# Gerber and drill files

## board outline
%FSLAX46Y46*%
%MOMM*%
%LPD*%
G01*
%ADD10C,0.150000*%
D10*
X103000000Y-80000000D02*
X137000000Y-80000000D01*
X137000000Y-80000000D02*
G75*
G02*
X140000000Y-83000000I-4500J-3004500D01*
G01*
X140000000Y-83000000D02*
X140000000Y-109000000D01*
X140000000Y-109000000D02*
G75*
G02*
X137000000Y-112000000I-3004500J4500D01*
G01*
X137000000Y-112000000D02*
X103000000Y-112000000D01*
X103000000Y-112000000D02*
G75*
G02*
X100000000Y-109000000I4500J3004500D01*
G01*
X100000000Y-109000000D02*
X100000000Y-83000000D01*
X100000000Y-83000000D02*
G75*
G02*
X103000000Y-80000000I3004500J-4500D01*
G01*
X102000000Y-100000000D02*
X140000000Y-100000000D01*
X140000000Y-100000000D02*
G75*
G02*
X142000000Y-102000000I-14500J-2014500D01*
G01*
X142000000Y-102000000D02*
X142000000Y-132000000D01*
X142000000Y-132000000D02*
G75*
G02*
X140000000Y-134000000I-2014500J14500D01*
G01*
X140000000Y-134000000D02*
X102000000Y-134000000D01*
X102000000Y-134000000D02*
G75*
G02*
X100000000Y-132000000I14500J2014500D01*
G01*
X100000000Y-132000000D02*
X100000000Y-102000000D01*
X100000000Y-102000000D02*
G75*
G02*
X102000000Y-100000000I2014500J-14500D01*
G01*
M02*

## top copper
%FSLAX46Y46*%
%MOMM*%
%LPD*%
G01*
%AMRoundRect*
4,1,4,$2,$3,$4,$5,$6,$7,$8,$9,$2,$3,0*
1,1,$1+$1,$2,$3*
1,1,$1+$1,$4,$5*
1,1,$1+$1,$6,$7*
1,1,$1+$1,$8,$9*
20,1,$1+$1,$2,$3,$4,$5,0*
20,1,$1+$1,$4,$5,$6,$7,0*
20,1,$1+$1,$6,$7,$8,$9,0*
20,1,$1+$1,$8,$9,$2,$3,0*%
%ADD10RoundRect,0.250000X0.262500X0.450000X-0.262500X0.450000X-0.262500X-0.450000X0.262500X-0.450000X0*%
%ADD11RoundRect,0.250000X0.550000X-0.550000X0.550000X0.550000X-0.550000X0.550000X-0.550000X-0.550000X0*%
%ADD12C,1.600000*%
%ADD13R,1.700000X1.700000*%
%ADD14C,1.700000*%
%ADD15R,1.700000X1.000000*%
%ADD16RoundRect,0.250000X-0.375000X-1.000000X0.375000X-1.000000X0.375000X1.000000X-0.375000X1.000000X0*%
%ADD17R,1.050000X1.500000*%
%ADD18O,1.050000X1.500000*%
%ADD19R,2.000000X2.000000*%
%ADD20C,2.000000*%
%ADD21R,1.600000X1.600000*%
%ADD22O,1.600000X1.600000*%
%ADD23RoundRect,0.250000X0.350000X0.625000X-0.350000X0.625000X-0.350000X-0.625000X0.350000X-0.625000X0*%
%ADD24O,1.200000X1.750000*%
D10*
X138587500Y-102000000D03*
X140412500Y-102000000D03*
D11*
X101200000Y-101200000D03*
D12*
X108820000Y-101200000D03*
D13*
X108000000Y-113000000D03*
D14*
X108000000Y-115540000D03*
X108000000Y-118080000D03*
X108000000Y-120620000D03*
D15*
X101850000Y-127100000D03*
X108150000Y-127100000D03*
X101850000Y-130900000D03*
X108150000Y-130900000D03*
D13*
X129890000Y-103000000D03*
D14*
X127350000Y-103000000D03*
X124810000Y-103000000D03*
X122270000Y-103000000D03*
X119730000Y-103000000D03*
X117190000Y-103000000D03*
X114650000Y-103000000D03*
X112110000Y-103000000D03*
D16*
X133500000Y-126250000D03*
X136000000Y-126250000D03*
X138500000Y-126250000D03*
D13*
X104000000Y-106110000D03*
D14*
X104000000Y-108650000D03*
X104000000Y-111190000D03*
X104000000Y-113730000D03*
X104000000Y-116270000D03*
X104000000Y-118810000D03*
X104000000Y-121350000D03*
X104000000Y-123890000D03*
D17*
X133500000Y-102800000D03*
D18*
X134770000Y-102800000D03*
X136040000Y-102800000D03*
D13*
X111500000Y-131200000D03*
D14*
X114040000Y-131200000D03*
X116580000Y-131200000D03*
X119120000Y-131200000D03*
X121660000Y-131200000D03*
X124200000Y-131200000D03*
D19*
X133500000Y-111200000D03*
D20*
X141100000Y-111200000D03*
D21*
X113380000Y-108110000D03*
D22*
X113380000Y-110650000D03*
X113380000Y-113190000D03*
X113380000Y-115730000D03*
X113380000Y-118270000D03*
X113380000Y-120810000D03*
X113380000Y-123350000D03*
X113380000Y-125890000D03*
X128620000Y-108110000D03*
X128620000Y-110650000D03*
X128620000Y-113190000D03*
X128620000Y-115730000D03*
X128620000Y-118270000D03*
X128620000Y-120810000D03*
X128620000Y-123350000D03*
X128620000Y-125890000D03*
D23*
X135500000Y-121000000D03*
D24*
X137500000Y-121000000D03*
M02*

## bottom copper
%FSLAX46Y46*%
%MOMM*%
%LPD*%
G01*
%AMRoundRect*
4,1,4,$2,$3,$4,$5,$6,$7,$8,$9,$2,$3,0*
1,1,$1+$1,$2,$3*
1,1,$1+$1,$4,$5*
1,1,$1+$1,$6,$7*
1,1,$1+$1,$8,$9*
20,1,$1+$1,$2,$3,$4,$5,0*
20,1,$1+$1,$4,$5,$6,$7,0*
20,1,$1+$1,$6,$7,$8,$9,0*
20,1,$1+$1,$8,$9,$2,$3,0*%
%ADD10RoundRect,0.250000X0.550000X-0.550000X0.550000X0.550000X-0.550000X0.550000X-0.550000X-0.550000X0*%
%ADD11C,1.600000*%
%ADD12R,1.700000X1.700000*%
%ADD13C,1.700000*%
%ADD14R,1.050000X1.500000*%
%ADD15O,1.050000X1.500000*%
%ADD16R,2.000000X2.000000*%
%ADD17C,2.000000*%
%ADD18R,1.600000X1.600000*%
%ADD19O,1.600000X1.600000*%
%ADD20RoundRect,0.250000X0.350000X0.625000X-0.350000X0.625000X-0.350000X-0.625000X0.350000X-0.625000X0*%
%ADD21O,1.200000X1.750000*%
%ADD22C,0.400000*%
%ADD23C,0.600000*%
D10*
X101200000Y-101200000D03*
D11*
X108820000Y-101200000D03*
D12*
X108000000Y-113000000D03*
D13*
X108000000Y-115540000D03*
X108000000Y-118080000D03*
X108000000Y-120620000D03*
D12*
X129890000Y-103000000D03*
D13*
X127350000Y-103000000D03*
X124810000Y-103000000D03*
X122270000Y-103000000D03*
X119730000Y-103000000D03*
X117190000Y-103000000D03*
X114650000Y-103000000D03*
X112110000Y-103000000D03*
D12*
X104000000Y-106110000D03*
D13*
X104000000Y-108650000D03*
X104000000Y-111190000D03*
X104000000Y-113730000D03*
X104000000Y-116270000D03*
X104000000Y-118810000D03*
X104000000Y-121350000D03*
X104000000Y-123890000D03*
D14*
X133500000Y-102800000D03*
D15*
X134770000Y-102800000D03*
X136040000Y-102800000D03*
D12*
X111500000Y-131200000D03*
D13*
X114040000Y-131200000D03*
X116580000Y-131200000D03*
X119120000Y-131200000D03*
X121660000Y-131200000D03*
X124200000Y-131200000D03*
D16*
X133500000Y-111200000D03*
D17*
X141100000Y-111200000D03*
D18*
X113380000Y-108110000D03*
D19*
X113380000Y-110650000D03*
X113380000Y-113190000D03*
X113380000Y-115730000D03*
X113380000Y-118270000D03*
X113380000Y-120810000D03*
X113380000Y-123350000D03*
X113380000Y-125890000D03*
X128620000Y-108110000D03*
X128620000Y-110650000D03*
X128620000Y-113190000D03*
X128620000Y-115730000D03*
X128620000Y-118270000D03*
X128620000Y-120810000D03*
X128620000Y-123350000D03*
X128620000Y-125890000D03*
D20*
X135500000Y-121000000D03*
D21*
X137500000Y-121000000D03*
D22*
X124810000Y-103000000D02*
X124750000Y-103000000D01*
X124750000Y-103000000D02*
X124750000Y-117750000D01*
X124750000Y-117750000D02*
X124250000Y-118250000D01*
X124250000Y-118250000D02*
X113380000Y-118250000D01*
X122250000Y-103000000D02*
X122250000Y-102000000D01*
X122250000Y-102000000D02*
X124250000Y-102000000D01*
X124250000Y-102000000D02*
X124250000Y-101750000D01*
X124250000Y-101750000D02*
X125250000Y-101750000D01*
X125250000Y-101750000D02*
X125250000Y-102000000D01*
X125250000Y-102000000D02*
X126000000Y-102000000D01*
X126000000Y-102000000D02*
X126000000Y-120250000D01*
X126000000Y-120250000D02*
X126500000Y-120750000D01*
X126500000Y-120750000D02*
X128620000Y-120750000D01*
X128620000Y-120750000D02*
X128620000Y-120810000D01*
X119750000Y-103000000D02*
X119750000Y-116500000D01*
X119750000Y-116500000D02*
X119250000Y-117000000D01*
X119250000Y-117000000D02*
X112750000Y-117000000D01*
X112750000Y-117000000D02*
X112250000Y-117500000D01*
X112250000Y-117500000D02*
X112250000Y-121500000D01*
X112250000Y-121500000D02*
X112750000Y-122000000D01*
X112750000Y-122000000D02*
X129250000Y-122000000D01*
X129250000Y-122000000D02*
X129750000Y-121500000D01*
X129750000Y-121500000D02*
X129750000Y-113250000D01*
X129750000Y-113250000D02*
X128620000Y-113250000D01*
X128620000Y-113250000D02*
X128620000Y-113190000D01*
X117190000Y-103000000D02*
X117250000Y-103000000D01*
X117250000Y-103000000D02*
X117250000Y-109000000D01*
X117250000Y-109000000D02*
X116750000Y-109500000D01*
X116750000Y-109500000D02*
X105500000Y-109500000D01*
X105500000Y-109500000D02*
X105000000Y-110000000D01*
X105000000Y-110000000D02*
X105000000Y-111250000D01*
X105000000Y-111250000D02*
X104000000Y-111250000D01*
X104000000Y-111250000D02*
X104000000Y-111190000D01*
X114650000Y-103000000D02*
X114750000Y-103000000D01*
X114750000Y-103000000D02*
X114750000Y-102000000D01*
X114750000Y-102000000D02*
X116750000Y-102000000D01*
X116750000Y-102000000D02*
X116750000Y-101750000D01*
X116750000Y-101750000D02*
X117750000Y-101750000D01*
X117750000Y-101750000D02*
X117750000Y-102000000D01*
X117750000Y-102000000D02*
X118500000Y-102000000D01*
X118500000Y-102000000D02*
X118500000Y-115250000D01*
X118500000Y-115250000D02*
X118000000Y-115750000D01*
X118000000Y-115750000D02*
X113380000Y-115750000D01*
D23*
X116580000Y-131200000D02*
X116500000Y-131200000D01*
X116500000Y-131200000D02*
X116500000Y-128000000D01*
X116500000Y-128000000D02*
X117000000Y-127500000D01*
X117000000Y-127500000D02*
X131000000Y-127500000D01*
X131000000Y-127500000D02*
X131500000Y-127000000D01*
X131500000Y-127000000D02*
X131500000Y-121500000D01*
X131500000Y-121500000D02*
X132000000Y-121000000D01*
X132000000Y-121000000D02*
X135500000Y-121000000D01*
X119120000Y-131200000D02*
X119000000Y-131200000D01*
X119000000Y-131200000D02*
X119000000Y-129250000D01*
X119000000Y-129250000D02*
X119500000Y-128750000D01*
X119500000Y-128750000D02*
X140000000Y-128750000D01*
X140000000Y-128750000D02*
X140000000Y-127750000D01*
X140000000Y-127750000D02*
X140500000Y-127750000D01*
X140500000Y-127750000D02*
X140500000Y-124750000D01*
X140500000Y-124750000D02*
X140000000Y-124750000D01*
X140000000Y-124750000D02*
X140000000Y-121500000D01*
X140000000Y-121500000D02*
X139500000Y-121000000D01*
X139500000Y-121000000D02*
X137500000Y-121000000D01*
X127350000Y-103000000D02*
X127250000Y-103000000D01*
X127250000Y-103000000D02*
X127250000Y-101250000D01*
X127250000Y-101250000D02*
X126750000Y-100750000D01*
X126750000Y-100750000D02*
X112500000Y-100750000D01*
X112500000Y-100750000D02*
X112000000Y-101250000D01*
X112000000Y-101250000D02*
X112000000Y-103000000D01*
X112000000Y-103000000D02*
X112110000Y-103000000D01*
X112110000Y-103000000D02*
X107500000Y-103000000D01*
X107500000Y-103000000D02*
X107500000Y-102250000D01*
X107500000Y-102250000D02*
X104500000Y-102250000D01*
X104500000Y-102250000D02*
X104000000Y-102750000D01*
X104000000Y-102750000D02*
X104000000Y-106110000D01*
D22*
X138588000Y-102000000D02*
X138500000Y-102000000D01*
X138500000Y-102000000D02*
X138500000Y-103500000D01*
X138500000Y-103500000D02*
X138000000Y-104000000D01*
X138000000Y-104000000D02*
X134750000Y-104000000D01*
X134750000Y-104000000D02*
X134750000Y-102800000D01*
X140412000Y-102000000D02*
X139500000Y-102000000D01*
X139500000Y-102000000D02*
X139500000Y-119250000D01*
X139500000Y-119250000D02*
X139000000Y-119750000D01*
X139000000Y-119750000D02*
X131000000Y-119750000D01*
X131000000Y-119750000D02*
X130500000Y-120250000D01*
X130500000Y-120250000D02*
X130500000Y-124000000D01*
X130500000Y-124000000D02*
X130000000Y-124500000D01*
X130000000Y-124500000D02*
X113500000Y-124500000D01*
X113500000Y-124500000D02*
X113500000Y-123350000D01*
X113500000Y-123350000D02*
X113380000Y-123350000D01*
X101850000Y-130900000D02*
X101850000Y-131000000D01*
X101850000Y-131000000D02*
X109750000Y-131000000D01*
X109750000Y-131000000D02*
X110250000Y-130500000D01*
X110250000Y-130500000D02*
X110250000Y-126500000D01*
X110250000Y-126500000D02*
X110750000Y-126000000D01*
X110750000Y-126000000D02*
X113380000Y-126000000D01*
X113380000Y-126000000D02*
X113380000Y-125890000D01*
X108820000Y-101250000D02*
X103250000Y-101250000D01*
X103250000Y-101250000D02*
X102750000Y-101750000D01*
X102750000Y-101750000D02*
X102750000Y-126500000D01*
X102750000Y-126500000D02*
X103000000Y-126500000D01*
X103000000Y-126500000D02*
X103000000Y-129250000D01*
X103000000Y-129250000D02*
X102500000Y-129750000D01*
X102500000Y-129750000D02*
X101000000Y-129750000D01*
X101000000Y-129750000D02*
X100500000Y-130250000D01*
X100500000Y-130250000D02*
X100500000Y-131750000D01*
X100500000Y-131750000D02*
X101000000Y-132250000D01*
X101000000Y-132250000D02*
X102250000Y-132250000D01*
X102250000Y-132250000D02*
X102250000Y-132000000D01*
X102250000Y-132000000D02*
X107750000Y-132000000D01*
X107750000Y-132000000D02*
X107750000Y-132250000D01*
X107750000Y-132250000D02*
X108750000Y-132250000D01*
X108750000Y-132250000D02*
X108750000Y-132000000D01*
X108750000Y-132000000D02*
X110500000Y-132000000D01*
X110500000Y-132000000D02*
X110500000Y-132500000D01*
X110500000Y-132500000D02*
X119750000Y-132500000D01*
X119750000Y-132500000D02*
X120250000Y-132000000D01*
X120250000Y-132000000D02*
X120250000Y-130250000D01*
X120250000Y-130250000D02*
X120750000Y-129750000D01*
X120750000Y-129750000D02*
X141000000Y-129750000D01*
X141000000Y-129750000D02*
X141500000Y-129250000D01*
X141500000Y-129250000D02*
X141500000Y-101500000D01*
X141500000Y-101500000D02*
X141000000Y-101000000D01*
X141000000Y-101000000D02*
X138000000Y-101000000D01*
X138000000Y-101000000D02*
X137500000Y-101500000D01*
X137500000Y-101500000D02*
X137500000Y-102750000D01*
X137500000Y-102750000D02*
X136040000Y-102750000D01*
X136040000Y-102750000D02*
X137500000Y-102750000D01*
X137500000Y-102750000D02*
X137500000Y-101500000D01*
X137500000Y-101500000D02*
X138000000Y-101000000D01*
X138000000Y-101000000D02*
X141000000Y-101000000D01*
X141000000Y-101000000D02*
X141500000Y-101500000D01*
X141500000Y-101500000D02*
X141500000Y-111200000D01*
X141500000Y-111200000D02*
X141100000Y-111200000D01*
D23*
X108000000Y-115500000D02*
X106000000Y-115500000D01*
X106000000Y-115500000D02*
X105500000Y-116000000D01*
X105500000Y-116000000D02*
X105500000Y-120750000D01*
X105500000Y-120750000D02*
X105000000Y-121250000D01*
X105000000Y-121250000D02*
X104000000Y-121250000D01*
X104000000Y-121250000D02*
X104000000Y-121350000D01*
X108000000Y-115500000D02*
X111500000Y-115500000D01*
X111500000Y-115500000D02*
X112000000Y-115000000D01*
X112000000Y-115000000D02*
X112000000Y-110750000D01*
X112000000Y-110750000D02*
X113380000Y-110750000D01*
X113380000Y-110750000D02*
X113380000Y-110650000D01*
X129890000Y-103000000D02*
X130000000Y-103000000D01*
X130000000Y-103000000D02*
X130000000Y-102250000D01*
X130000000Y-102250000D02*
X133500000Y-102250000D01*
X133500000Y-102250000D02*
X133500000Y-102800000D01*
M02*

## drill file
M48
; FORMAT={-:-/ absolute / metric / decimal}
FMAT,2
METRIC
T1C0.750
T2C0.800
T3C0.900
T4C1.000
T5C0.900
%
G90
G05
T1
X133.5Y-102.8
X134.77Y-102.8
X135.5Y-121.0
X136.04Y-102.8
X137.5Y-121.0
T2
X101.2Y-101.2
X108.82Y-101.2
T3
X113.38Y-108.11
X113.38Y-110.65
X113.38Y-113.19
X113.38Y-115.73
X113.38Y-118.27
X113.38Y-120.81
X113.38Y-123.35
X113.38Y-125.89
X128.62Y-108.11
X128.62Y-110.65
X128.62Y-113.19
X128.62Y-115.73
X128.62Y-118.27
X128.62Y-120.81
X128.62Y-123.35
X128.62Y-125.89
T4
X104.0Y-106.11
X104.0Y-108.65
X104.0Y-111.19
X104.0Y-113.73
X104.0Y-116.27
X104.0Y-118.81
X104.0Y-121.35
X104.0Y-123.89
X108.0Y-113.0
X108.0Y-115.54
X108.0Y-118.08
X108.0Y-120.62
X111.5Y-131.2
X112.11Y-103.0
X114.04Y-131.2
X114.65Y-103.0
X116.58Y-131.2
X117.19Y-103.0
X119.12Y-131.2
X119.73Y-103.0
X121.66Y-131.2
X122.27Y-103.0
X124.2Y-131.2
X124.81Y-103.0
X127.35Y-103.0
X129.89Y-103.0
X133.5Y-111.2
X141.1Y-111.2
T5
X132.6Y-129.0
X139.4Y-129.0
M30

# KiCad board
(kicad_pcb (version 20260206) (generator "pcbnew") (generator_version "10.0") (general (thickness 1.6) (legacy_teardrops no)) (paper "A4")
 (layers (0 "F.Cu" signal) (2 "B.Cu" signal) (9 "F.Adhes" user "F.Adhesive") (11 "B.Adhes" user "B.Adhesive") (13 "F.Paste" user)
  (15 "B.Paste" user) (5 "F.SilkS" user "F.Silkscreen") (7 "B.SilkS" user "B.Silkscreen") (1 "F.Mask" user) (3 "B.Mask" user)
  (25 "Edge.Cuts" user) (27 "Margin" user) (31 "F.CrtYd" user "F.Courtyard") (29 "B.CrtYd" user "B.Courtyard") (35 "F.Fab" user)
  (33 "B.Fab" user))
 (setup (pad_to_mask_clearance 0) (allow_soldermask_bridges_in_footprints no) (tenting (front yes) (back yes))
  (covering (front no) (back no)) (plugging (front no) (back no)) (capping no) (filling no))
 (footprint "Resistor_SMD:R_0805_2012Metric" (layer "F.Cu") (at 139.50 102.00 0)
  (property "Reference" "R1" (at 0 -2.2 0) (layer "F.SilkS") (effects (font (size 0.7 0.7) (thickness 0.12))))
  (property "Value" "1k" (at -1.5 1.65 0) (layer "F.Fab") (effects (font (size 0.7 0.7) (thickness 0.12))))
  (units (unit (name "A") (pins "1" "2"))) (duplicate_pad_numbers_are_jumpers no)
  (pad "1" smd roundrect (at -0.9125 0 180) (size 1.025 1.4) (layers "F.Cu" "F.Mask" "F.Paste") (roundrect_rratio 0.243902)
   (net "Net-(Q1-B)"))
  (pad "2" smd roundrect (at 0.9125 0 180) (size 1.025 1.4) (layers "F.Cu" "F.Mask" "F.Paste") (roundrect_rratio 0.243902)
   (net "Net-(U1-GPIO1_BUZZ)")))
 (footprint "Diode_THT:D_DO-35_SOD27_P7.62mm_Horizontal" (layer "F.Cu") (at 101.20 101.20 0)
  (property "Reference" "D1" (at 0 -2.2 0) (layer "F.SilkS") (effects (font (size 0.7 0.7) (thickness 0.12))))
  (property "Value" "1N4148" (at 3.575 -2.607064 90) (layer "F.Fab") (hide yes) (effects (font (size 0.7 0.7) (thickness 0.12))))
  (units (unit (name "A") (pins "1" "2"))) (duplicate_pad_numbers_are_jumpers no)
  (pad "1" thru_hole roundrect (at 0 0 90) (size 1.6 1.6) (drill 0.8) (layers "*.Cu" "*.Mask") (remove_unused_layers no)
   (roundrect_rratio 0.15625) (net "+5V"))
  (pad "2" thru_hole circle (at 7.62 0 90) (size 1.6 1.6) (drill 0.8) (layers "*.Cu" "*.Mask") (remove_unused_layers no) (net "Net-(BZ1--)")))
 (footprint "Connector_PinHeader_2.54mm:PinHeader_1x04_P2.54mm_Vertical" (layer "F.Cu") (at 108.00 113.00 0)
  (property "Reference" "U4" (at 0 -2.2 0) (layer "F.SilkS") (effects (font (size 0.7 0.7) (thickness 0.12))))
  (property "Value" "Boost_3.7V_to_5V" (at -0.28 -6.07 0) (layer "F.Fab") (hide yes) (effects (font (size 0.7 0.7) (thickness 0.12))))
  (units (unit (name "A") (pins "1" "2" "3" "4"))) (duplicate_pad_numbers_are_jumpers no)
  (pad "1" thru_hole rect (at 0 0 180) (size 1.7 1.7) (drill 1) (layers "*.Cu" "*.Mask") (remove_unused_layers no) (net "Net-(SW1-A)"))
  (pad "2" thru_hole circle (at 0 2.54 180) (size 1.7 1.7) (drill 1) (layers "*.Cu" "*.Mask") (remove_unused_layers no) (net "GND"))
  (pad "3" thru_hole circle (at 0 5.08 180) (size 1.7 1.7) (drill 1) (layers "*.Cu" "*.Mask") (remove_unused_layers no)
   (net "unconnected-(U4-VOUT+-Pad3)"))
  (pad "4" thru_hole circle (at 0 7.62 180) (size 1.7 1.7) (drill 1) (layers "*.Cu" "*.Mask") (remove_unused_layers no)
   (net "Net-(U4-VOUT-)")))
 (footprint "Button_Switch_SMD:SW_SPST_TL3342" (layer "F.Cu") (at 105.00 129.00 0)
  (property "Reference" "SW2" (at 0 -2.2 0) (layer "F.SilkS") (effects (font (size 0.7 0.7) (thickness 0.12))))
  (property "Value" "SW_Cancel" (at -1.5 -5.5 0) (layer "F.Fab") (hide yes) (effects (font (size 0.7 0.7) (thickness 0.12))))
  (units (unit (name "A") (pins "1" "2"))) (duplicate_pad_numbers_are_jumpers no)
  (pad "1" smd rect (at -3.15 -1.9) (size 1.7 1) (layers "F.Cu" "F.Mask" "F.Paste") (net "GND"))
  (pad "1" smd rect (at 3.15 -1.9) (size 1.7 1) (layers "F.Cu" "F.Mask" "F.Paste") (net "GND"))
  (pad "2" smd rect (at -3.15 1.9) (size 1.7 1) (layers "F.Cu" "F.Mask" "F.Paste") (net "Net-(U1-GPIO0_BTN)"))
  (pad "2" smd rect (at 3.15 1.9) (size 1.7 1) (layers "F.Cu" "F.Mask" "F.Paste") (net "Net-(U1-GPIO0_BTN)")))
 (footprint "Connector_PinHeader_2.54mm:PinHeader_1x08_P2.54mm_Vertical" (layer "F.Cu") (at 129.89 103.00 -90)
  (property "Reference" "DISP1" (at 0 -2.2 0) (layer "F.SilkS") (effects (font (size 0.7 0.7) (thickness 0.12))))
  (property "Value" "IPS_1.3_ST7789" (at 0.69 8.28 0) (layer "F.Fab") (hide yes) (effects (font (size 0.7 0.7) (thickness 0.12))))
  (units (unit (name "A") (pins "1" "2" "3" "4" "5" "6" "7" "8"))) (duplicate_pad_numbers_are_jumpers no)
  (pad "1" thru_hole rect (at 0 0 270) (size 1.7 1.7) (drill 1) (layers "*.Cu" "*.Mask") (remove_unused_layers no) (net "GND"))
  (pad "2" thru_hole circle (at 0 2.54 270) (size 1.7 1.7) (drill 1) (layers "*.Cu" "*.Mask") (remove_unused_layers no) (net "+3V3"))
  (pad "3" thru_hole circle (at 0 5.08 270) (size 1.7 1.7) (drill 1) (layers "*.Cu" "*.Mask") (remove_unused_layers no)
   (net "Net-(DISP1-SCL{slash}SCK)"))
  (pad "4" thru_hole circle (at 0 7.62 270) (size 1.7 1.7) (drill 1) (layers "*.Cu" "*.Mask") (remove_unused_layers no)
   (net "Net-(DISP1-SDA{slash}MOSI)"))
  (pad "5" thru_hole circle (at 0 10.16 270) (size 1.7 1.7) (drill 1) (layers "*.Cu" "*.Mask") (remove_unused_layers no)
   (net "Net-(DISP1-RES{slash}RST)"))
  (pad "6" thru_hole circle (at 0 12.7 270) (size 1.7 1.7) (drill 1) (layers "*.Cu" "*.Mask") (remove_unused_layers no)
   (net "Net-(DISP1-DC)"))
  (pad "7" thru_hole circle (at 0 15.24 270) (size 1.7 1.7) (drill 1) (layers "*.Cu" "*.Mask") (remove_unused_layers no)
   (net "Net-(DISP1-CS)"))
  (pad "8" thru_hole circle (at 0 17.78 270) (size 1.7 1.7) (drill 1) (layers "*.Cu" "*.Mask") (remove_unused_layers no) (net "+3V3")))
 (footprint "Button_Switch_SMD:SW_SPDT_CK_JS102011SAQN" (layer "F.Cu") (at 136.00 129.00 0)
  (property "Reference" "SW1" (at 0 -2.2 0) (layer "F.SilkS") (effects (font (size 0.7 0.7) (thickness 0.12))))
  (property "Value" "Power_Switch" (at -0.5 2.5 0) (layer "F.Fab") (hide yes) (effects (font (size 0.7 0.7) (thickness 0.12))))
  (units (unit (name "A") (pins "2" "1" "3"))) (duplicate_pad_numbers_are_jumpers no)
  (pad "" np_thru_hole circle (at -3.4 0) (size 0.9 0.9) (drill 0.9) (layers "*.Cu" "*.Mask"))
  (pad "" np_thru_hole circle (at 3.4 0) (size 0.9 0.9) (drill 0.9) (layers "*.Cu" "*.Mask"))
  (pad "1" smd roundrect (at -2.5 -2.75) (size 1.25 2.5) (layers "F.Cu" "F.Mask" "F.Paste") (roundrect_rratio 0.2) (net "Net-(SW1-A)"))
  (pad "2" smd roundrect (at 0 -2.75) (size 1.25 2.5) (layers "F.Cu" "F.Mask" "F.Paste") (roundrect_rratio 0.2) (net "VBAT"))
  (pad "3" smd roundrect (at 2.5 -2.75) (size 1.25 2.5) (layers "F.Cu" "F.Mask" "F.Paste") (roundrect_rratio 0.2)
   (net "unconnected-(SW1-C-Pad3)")))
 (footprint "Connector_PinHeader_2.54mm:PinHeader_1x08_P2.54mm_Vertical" (layer "F.Cu") (at 104.00 106.11 0)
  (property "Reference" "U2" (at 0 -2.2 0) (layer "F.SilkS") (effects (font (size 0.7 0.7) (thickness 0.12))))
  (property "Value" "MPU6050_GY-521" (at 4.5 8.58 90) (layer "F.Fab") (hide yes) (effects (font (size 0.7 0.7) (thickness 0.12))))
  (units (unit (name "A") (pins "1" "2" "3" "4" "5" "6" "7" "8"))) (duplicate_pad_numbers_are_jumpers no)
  (pad "1" thru_hole rect (at 0 0) (size 1.7 1.7) (drill 1) (layers "*.Cu" "*.Mask") (remove_unused_layers no) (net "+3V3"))
  (pad "2" thru_hole circle (at 0 2.54) (size 1.7 1.7) (drill 1) (layers "*.Cu" "*.Mask") (remove_unused_layers no) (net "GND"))
  (pad "3" thru_hole circle (at 0 5.08) (size 1.7 1.7) (drill 1) (layers "*.Cu" "*.Mask") (remove_unused_layers no) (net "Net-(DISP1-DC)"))
  (pad "4" thru_hole circle (at 0 7.62) (size 1.7 1.7) (drill 1) (layers "*.Cu" "*.Mask") (remove_unused_layers no)
   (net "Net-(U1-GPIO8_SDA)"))
  (pad "5" thru_hole circle (at 0 10.16) (size 1.7 1.7) (drill 1) (layers "*.Cu" "*.Mask") (remove_unused_layers no)
   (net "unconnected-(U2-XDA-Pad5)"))
  (pad "6" thru_hole circle (at 0 12.7) (size 1.7 1.7) (drill 1) (layers "*.Cu" "*.Mask") (remove_unused_layers no)
   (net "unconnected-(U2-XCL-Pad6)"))
  (pad "7" thru_hole circle (at 0 15.24) (size 1.7 1.7) (drill 1) (layers "*.Cu" "*.Mask") (remove_unused_layers no) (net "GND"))
  (pad "8" thru_hole circle (at 0 17.78) (size 1.7 1.7) (drill 1) (layers "*.Cu" "*.Mask") (remove_unused_layers no)
   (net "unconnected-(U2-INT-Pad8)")))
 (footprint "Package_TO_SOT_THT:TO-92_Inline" (layer "F.Cu") (at 133.50 102.80 0)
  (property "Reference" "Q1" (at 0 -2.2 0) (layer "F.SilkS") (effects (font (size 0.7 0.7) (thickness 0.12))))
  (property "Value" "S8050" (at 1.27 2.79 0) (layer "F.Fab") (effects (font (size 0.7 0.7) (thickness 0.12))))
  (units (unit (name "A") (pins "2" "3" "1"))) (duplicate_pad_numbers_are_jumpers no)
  (pad "1" thru_hole rect (at 0 0) (size 1.05 1.5) (drill 0.75) (layers "*.Cu" "*.Mask") (remove_unused_layers no) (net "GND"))
  (pad "2" thru_hole oval (at 1.27 0) (size 1.05 1.5) (drill 0.75) (layers "*.Cu" "*.Mask") (remove_unused_layers no) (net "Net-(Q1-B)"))
  (pad "3" thru_hole oval (at 2.54 0) (size 1.05 1.5) (drill 0.75) (layers "*.Cu" "*.Mask") (remove_unused_layers no) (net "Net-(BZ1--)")))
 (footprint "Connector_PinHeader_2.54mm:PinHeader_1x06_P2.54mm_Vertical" (layer "F.Cu") (at 111.50 131.20 90)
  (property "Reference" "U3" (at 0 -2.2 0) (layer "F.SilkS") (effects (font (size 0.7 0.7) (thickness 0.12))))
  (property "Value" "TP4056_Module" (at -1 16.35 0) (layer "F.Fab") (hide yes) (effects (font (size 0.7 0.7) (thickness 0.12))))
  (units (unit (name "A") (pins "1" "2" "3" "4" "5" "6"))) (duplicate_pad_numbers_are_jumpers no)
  (pad "1" thru_hole rect (at 0 0) (size 1.7 1.7) (drill 1) (layers "*.Cu" "*.Mask") (remove_unused_layers no)
   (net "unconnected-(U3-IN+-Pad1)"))
  (pad "2" thru_hole circle (at 0 2.54) (size 1.7 1.7) (drill 1) (layers "*.Cu" "*.Mask") (remove_unused_layers no)
   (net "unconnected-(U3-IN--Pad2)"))
  (pad "3" thru_hole circle (at 0 5.08) (size 1.7 1.7) (drill 1) (layers "*.Cu" "*.Mask") (remove_unused_layers no) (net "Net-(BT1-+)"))
  (pad "4" thru_hole circle (at 0 7.62) (size 1.7 1.7) (drill 1) (layers "*.Cu" "*.Mask") (remove_unused_layers no) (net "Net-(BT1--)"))
  (pad "5" thru_hole circle (at 0 10.16) (size 1.7 1.7) (drill 1) (layers "*.Cu" "*.Mask") (remove_unused_layers no) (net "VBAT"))
  (pad "6" thru_hole circle (at 0 12.7) (size 1.7 1.7) (drill 1) (layers "*.Cu" "*.Mask") (remove_unused_layers no) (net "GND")))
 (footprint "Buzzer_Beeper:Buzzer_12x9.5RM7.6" (layer "F.Cu") (at 133.50 111.20 0)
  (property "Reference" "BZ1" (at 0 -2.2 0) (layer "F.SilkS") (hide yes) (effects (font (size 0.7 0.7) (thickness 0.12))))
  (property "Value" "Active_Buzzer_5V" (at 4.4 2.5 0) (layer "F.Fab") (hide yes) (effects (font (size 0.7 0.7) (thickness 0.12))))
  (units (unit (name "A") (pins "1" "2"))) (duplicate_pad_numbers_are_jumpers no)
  (pad "1" thru_hole rect (at 0 0) (size 2 2) (drill 1) (layers "*.Cu" "*.Mask") (remove_unused_layers no) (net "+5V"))
  (pad "2" thru_hole circle (at 7.6 0) (size 2 2) (drill 1) (layers "*.Cu" "*.Mask") (remove_unused_layers no) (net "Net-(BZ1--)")))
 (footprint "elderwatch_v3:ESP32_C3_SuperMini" (layer "F.Cu") (at 121.00 117.00 0)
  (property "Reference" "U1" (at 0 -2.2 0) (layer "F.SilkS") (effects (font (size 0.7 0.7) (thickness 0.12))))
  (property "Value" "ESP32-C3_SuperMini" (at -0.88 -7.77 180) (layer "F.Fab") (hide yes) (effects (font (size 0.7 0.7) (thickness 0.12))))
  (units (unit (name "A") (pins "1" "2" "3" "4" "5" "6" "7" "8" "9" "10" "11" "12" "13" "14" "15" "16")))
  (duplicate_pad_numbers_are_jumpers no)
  (pad "1" thru_hole rect (at -7.62 -8.89 180) (size 1.6 1.6) (drill 0.9) (layers "*.Cu" "*.Mask") (remove_unused_layers no)
   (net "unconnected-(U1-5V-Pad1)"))
  (pad "2" thru_hole oval (at -7.62 -6.35 180) (size 1.6 1.6) (drill 0.9) (layers "*.Cu" "*.Mask") (remove_unused_layers no) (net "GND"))
  (pad "3" thru_hole oval (at -7.62 -3.81 180) (size 1.6 1.6) (drill 0.9) (layers "*.Cu" "*.Mask") (remove_unused_layers no)
   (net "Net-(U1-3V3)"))
  (pad "4" thru_hole oval (at -7.62 -1.27 180) (size 1.6 1.6) (drill 0.9) (layers "*.Cu" "*.Mask") (remove_unused_layers no)
   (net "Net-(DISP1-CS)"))
  (pad "5" thru_hole oval (at -7.62 1.27 180) (size 1.6 1.6) (drill 0.9) (layers "*.Cu" "*.Mask") (remove_unused_layers no)
   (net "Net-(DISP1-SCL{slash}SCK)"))
  (pad "6" thru_hole oval (at -7.62 3.81 180) (size 1.6 1.6) (drill 0.9) (layers "*.Cu" "*.Mask") (remove_unused_layers no)
   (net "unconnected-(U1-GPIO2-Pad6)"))
  (pad "7" thru_hole oval (at -7.62 6.35 180) (size 1.6 1.6) (drill 0.9) (layers "*.Cu" "*.Mask") (remove_unused_layers no)
   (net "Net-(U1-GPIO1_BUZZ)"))
  (pad "8" thru_hole oval (at -7.62 8.89 180) (size 1.6 1.6) (drill 0.9) (layers "*.Cu" "*.Mask") (remove_unused_layers no)
   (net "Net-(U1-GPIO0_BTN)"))
  (pad "9" thru_hole oval (at 7.62 -8.89 180) (size 1.6 1.6) (drill 0.9) (layers "*.Cu" "*.Mask") (remove_unused_layers no)
   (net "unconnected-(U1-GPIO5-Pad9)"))
  (pad "10" thru_hole oval (at 7.62 -6.35 180) (size 1.6 1.6) (drill 0.9) (layers "*.Cu" "*.Mask") (remove_unused_layers no)
   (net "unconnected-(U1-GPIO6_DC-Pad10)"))
  (pad "11" thru_hole oval (at 7.62 -3.81 180) (size 1.6 1.6) (drill 0.9) (layers "*.Cu" "*.Mask") (remove_unused_layers no)
   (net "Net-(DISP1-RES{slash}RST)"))
  (pad "12" thru_hole oval (at 7.62 -1.27 180) (size 1.6 1.6) (drill 0.9) (layers "*.Cu" "*.Mask") (remove_unused_layers no)
   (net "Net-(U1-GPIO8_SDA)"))
  (pad "13" thru_hole oval (at 7.62 1.27 180) (size 1.6 1.6) (drill 0.9) (layers "*.Cu" "*.Mask") (remove_unused_layers no)
   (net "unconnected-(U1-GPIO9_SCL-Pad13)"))
  (pad "14" thru_hole oval (at 7.62 3.81 180) (size 1.6 1.6) (drill 0.9) (layers "*.Cu" "*.Mask") (remove_unused_layers no)
   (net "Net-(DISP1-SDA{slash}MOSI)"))
  (pad "15" thru_hole oval (at 7.62 6.35 180) (size 1.6 1.6) (drill 0.9) (layers "*.Cu" "*.Mask") (remove_unused_layers no)
   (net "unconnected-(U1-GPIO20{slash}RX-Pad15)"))
  (pad "16" thru_hole oval (at 7.62 8.89 180) (size 1.6 1.6) (drill 0.9) (layers "*.Cu" "*.Mask") (remove_unused_layers no)
   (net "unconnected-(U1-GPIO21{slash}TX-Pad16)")))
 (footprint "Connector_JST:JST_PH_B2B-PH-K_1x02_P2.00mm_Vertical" (layer "F.Cu") (at 135.50 121.00 0)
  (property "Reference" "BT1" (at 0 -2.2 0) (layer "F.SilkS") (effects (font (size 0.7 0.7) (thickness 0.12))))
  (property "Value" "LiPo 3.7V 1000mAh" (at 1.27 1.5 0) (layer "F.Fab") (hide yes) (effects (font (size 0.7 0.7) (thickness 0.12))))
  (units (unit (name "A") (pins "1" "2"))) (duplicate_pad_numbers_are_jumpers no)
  (pad "1" thru_hole roundrect (at 0 0 180) (size 1.2 1.75) (drill 0.75) (layers "*.Cu" "*.Mask") (remove_unused_layers no)
   (roundrect_rratio 0.208333) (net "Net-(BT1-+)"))
  (pad "2" thru_hole oval (at 2 0 180) (size 1.2 1.75) (drill 0.75) (layers "*.Cu" "*.Mask") (remove_unused_layers no) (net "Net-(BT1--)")))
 (gr_line (start 103.0 80.0) (end 137.0 80.0) (stroke (width 0.15) (type default)) (layer "Edge.Cuts"))
 (gr_arc (start 137.0 80.0) (mid 139.12 80.88) (end 140.0 83.0) (stroke (width 0.15) (type default)) (layer "Edge.Cuts"))
 (gr_line (start 140.0 83.0) (end 140.0 109.0) (stroke (width 0.15) (type default)) (layer "Edge.Cuts"))
 (gr_arc (start 140.0 109.0) (mid 139.12 111.12) (end 137.0 112.0) (stroke (width 0.15) (type default)) (layer "Edge.Cuts"))
 (gr_line (start 137.0 112.0) (end 103.0 112.0) (stroke (width 0.15) (type default)) (layer "Edge.Cuts"))
 (gr_arc (start 103.0 112.0) (mid 100.88 111.12) (end 100.0 109.0) (stroke (width 0.15) (type default)) (layer "Edge.Cuts"))
 (gr_line (start 100.0 109.0) (end 100.0 83.0) (stroke (width 0.15) (type default)) (layer "Edge.Cuts"))
 (gr_arc (start 100.0 83.0) (mid 100.88 80.88) (end 103.0 80.0) (stroke (width 0.15) (type default)) (layer "Edge.Cuts"))
 (gr_line (start 102.0 100.0) (end 140.0 100.0) (stroke (width 0.15) (type default)) (layer "Edge.Cuts"))
 (gr_arc (start 140.0 100.0) (mid 141.41 100.59) (end 142.0 102.0) (stroke (width 0.15) (type default)) (layer "Edge.Cuts"))
 (gr_line (start 142.0 102.0) (end 142.0 132.0) (stroke (width 0.15) (type default)) (layer "Edge.Cuts"))
 (gr_arc (start 142.0 132.0) (mid 141.41 133.41) (end 140.0 134.0) (stroke (width 0.15) (type default)) (layer "Edge.Cuts"))
 (gr_line (start 140.0 134.0) (end 102.0 134.0) (stroke (width 0.15) (type default)) (layer "Edge.Cuts"))
 (gr_arc (start 102.0 134.0) (mid 100.59 133.41) (end 100.0 132.0) (stroke (width 0.15) (type default)) (layer "Edge.Cuts"))
 (gr_line (start 100.0 132.0) (end 100.0 102.0) (stroke (width 0.15) (type default)) (layer "Edge.Cuts"))
 (gr_arc (start 100.0 102.0) (mid 100.59 100.59) (end 102.0 100.0) (stroke (width 0.15) (type default)) (layer "Edge.Cuts"))
 (segment (start 124.810 103.000) (end 124.750 103.000) (width 0.40) (layer "B.Cu") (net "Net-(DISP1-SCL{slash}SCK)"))
 (segment (start 124.750 103.000) (end 124.750 117.750) (width 0.40) (layer "B.Cu") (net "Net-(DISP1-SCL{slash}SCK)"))
 (segment (start 124.750 117.750) (end 124.250 118.250) (width 0.40) (layer "B.Cu") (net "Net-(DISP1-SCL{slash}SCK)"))
 (segment (start 124.250 118.250) (end 113.380 118.250) (width 0.40) (layer "B.Cu") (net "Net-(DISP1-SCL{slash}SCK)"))
 (segment (start 122.250 103.000) (end 122.250 102.000) (width 0.40) (layer "B.Cu") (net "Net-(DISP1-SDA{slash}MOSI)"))
 (segment (start 122.250 102.000) (end 124.250 102.000) (width 0.40) (layer "B.Cu") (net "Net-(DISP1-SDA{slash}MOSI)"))
 (segment (start 124.250 102.000) (end 124.250 101.750) (width 0.40) (layer "B.Cu") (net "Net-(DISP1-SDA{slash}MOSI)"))
 (segment (start 124.250 101.750) (end 125.250 101.750) (width 0.40) (layer "B.Cu") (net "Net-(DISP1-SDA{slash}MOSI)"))
 (segment (start 125.250 101.750) (end 125.250 102.000) (width 0.40) (layer "B.Cu") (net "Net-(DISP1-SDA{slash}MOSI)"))
 (segment (start 125.250 102.000) (end 126.000 102.000) (width 0.40) (layer "B.Cu") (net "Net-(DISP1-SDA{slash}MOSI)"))
 (segment (start 126.000 102.000) (end 126.000 120.250) (width 0.40) (layer "B.Cu") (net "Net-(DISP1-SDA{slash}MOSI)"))
 (segment (start 126.000 120.250) (end 126.500 120.750) (width 0.40) (layer "B.Cu") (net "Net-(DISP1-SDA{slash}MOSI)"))
 (segment (start 126.500 120.750) (end 128.620 120.750) (width 0.40) (layer "B.Cu") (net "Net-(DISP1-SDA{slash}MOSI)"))
 (segment (start 128.620 120.750) (end 128.620 120.810) (width 0.40) (layer "B.Cu") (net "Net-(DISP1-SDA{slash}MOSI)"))
 (segment (start 119.750 103.000) (end 119.750 116.500) (width 0.40) (layer "B.Cu") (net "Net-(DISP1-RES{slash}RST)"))
 (segment (start 119.750 116.500) (end 119.250 117.000) (width 0.40) (layer "B.Cu") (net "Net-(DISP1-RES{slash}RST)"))
 (segment (start 119.250 117.000) (end 112.750 117.000) (width 0.40) (layer "B.Cu") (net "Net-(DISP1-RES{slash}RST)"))
 (segment (start 112.750 117.000) (end 112.250 117.500) (width 0.40) (layer "B.Cu") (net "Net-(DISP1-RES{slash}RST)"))
 (segment (start 112.250 117.500) (end 112.250 121.500) (width 0.40) (layer "B.Cu") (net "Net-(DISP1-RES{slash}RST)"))
 (segment (start 112.250 121.500) (end 112.750 122.000) (width 0.40) (layer "B.Cu") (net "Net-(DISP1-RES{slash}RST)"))
 (segment (start 112.750 122.000) (end 129.250 122.000) (width 0.40) (layer "B.Cu") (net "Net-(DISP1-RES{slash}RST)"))
 (segment (start 129.250 122.000) (end 129.750 121.500) (width 0.40) (layer "B.Cu") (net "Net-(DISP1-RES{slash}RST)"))
 (segment (start 129.750 121.500) (end 129.750 113.250) (width 0.40) (layer "B.Cu") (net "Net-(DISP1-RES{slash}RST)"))
 (segment (start 129.750 113.250) (end 128.620 113.250) (width 0.40) (layer "B.Cu") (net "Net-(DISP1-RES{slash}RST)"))
 (segment (start 128.620 113.250) (end 128.620 113.190) (width 0.40) (layer "B.Cu") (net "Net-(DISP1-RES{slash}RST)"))
 (segment (start 117.190 103.000) (end 117.250 103.000) (width 0.40) (layer "B.Cu") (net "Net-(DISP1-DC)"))
 (segment (start 117.250 103.000) (end 117.250 109.000) (width 0.40) (layer "B.Cu") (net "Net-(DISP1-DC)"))
 (segment (start 117.250 109.000) (end 116.750 109.500) (width 0.40) (layer "B.Cu") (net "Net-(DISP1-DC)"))
 (segment (start 116.750 109.500) (end 105.500 109.500) (width 0.40) (layer "B.Cu") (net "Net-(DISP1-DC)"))
 (segment (start 105.500 109.500) (end 105.000 110.000) (width 0.40) (layer "B.Cu") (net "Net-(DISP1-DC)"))
 (segment (start 105.000 110.000) (end 105.000 111.250) (width 0.40) (layer "B.Cu") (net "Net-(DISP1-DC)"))
 (segment (start 105.000 111.250) (end 104.000 111.250) (width 0.40) (layer "B.Cu") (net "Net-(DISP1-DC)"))
 (segment (start 104.000 111.250) (end 104.000 111.190) (width 0.40) (layer "B.Cu") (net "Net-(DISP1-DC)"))
 (segment (start 114.650 103.000) (end 114.750 103.000) (width 0.40) (layer "B.Cu") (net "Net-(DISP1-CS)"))
 (segment (start 114.750 103.000) (end 114.750 102.000) (width 0.40) (layer "B.Cu") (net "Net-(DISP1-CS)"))
 (segment (start 114.750 102.000) (end 116.750 102.000) (width 0.40) (layer "B.Cu") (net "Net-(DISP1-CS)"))
 (segment (start 116.750 102.000) (end 116.750 101.750) (width 0.40) (layer "B.Cu") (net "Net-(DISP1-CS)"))
 (segment (start 116.750 101.750) (end 117.750 101.750) (width 0.40) (layer "B.Cu") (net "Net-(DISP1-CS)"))
 (segment (start 117.750 101.750) (end 117.750 102.000) (width 0.40) (layer "B.Cu") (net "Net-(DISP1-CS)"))
 (segment (start 117.750 102.000) (end 118.500 102.000) (width 0.40) (layer "B.Cu") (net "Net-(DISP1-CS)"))
 (segment (start 118.500 102.000) (end 118.500 115.250) (width 0.40) (layer "B.Cu") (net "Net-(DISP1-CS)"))
 (segment (start 118.500 115.250) (end 118.000 115.750) (width 0.40) (layer "B.Cu") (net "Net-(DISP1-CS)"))
 (segment (start 118.000 115.750) (end 113.380 115.750) (width 0.40) (layer "B.Cu") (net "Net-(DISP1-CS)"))
 (segment (start 116.580 131.200) (end 116.500 131.200) (width 0.60) (layer "B.Cu") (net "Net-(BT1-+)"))
 (segment (start 116.500 131.200) (end 116.500 128.000) (width 0.60) (layer "B.Cu") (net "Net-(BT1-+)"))
 (segment (start 116.500 128.000) (end 117.000 127.500) (width 0.60) (layer "B.Cu") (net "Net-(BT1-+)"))
 (segment (start 117.000 127.500) (end 131.000 127.500) (width 0.60) (layer "B.Cu") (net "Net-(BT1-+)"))
 (segment (start 131.000 127.500) (end 131.500 127.000) (width 0.60) (layer "B.Cu") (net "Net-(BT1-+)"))
 (segment (start 131.500 127.000) (end 131.500 121.500) (width 0.60) (layer "B.Cu") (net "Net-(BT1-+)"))
 (segment (start 131.500 121.500) (end 132.000 121.000) (width 0.60) (layer "B.Cu") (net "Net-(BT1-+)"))
 (segment (start 132.000 121.000) (end 135.500 121.000) (width 0.60) (layer "B.Cu") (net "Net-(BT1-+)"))
 (segment (start 119.120 131.200) (end 119.000 131.200) (width 0.60) (layer "B.Cu") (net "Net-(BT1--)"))
 (segment (start 119.000 131.200) (end 119.000 129.250) (width 0.60) (layer "B.Cu") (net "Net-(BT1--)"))
 (segment (start 119.000 129.250) (end 119.500 128.750) (width 0.60) (layer "B.Cu") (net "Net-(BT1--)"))
 (segment (start 119.500 128.750) (end 140.000 128.750) (width 0.60) (layer "B.Cu") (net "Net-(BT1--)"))
 (segment (start 140.000 128.750) (end 140.000 127.750) (width 0.60) (layer "B.Cu") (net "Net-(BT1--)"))
 (segment (start 140.000 127.750) (end 140.500 127.750) (width 0.60) (layer "B.Cu") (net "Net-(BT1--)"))
 (segment (start 140.500 127.750) (end 140.500 124.750) (width 0.60) (layer "B.Cu") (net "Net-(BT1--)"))
 (segment (start 140.500 124.750) (end 140.000 124.750) (width 0.60) (layer "B.Cu") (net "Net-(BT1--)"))
 (segment (start 140.000 124.750) (end 140.000 121.500) (width 0.60) (layer "B.Cu") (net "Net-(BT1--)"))
 (segment (start 140.000 121.500) (end 139.500 121.000) (width 0.60) (layer "B.Cu") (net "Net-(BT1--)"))
 (segment (start 139.500 121.000) (end 137.500 121.000) (width 0.60) (layer "B.Cu") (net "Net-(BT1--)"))
 (segment (start 127.350 103.000) (end 127.250 103.000) (width 0.60) (layer "B.Cu") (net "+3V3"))
 (segment (start 127.250 103.000) (end 127.250 101.250) (width 0.60) (layer "B.Cu") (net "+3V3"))
 (segment (start 127.250 101.250) (end 126.750 100.750) (width 0.60) (layer "B.Cu") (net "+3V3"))
 (segment (start 126.750 100.750) (end 112.500 100.750) (width 0.60) (layer "B.Cu") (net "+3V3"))
 (segment (start 112.500 100.750) (end 112.000 101.250) (width 0.60) (layer "B.Cu") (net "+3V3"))
 (segment (start 112.000 101.250) (end 112.000 103.000) (width 0.60) (layer "B.Cu") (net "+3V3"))
 (segment (start 112.000 103.000) (end 112.110 103.000) (width 0.60) (layer "B.Cu") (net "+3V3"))
 (segment (start 112.110 103.000) (end 107.500 103.000) (width 0.60) (layer "B.Cu") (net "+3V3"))
 (segment (start 107.500 103.000) (end 107.500 102.250) (width 0.60) (layer "B.Cu") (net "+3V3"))
 (segment (start 107.500 102.250) (end 104.500 102.250) (width 0.60) (layer "B.Cu") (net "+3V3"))
 (segment (start 104.500 102.250) (end 104.000 102.750) (width 0.60) (layer "B.Cu") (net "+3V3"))
 (segment (start 104.000 102.750) (end 104.000 106.110) (width 0.60) (layer "B.Cu") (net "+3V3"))
 (segment (start 138.588 102.000) (end 138.500 102.000) (width 0.40) (layer "B.Cu") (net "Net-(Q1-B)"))
 (segment (start 138.500 102.000) (end 138.500 103.500) (width 0.40) (layer "B.Cu") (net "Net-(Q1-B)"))
 (segment (start 138.500 103.500) (end 138.000 104.000) (width 0.40) (layer "B.Cu") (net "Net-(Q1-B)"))
 (segment (start 138.000 104.000) (end 134.750 104.000) (width 0.40) (layer "B.Cu") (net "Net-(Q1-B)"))
 (segment (start 134.750 104.000) (end 134.750 102.800) (width 0.40) (layer "B.Cu") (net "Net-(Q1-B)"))
 (segment (start 140.412 102.000) (end 139.500 102.000) (width 0.40) (layer "B.Cu") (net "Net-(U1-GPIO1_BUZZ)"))
 (segment (start 139.500 102.000) (end 139.500 119.250) (width 0.40) (layer "B.Cu") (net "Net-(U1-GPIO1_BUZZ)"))
 (segment (start 139.500 119.250) (end 139.000 119.750) (width 0.40) (layer "B.Cu") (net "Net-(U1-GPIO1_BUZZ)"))
 (segment (start 139.000 119.750) (end 131.000 119.750) (width 0.40) (layer "B.Cu") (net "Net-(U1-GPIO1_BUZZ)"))
 (segment (start 131.000 119.750) (end 130.500 120.250) (width 0.40) (layer "B.Cu") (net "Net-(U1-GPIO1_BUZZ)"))
 (segment (start 130.500 120.250) (end 130.500 124.000) (width 0.40) (layer "B.Cu") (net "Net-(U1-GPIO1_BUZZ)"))
 (segment (start 130.500 124.000) (end 130.000 124.500) (width 0.40) (layer "B.Cu") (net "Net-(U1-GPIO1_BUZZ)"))
 (segment (start 130.000 124.500) (end 113.500 124.500) (width 0.40) (layer "B.Cu") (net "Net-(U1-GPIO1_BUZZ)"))
 (segment (start 113.500 124.500) (end 113.500 123.350) (width 0.40) (layer "B.Cu") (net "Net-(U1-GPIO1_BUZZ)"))
 (segment (start 113.500 123.350) (end 113.380 123.350) (width 0.40) (layer "B.Cu") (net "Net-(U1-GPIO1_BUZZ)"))
 (segment (start 101.850 130.900) (end 101.850 131.000) (width 0.40) (layer "B.Cu") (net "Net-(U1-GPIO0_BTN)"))
 (segment (start 101.850 131.000) (end 109.750 131.000) (width 0.40) (layer "B.Cu") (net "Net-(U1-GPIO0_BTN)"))
 (segment (start 109.750 131.000) (end 110.250 130.500) (width 0.40) (layer "B.Cu") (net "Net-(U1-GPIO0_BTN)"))
 (segment (start 110.250 130.500) (end 110.250 126.500) (width 0.40) (layer "B.Cu") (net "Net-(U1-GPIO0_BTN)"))
 (segment (start 110.250 126.500) (end 110.750 126.000) (width 0.40) (layer "B.Cu") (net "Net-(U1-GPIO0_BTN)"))
 (segment (start 110.750 126.000) (end 113.380 126.000) (width 0.40) (layer "B.Cu") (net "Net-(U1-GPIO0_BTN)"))
 (segment (start 113.380 126.000) (end 113.380 125.890) (width 0.40) (layer "B.Cu") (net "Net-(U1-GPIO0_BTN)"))
 (segment (start 108.820 101.250) (end 103.250 101.250) (width 0.40) (layer "B.Cu") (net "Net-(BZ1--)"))
 (segment (start 103.250 101.250) (end 102.750 101.750) (width 0.40) (layer "B.Cu") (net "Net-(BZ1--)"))
 (segment (start 102.750 101.750) (end 102.750 126.500) (width 0.40) (layer "B.Cu") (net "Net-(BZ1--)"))
 (segment (start 102.750 126.500) (end 103.000 126.500) (width 0.40) (layer "B.Cu") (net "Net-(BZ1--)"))
 (segment (start 103.000 126.500) (end 103.000 129.250) (width 0.40) (layer "B.Cu") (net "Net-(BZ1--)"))
 (segment (start 103.000 129.250) (end 102.500 129.750) (width 0.40) (layer "B.Cu") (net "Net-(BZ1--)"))
 (segment (start 102.500 129.750) (end 101.000 129.750) (width 0.40) (layer "B.Cu") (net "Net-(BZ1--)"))
 (segment (start 101.000 129.750) (end 100.500 130.250) (width 0.40) (layer "B.Cu") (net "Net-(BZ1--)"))
 (segment (start 100.500 130.250) (end 100.500 131.750) (width 0.40) (layer "B.Cu") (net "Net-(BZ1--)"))
 (segment (start 100.500 131.750) (end 101.000 132.250) (width 0.40) (layer "B.Cu") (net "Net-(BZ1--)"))
 (segment (start 101.000 132.250) (end 102.250 132.250) (width 0.40) (layer "B.Cu") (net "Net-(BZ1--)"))
 (segment (start 102.250 132.250) (end 102.250 132.000) (width 0.40) (layer "B.Cu") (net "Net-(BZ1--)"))
 (segment (start 102.250 132.000) (end 107.750 132.000) (width 0.40) (layer "B.Cu") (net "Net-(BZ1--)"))
 (segment (start 107.750 132.000) (end 107.750 132.250) (width 0.40) (layer "B.Cu") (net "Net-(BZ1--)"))
 (segment (start 107.750 132.250) (end 108.750 132.250) (width 0.40) (layer "B.Cu") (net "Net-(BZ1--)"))
 (segment (start 108.750 132.250) (end 108.750 132.000) (width 0.40) (layer "B.Cu") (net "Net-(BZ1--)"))
 (segment (start 108.750 132.000) (end 110.500 132.000) (width 0.40) (layer "B.Cu") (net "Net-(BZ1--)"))
 (segment (start 110.500 132.000) (end 110.500 132.500) (width 0.40) (layer "B.Cu") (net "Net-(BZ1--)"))
 (segment (start 110.500 132.500) (end 119.750 132.500) (width 0.40) (layer "B.Cu") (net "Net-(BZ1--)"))
 (segment (start 119.750 132.500) (end 120.250 132.000) (width 0.40) (layer "B.Cu") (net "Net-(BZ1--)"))
 (segment (start 120.250 132.000) (end 120.250 130.250) (width 0.40) (layer "B.Cu") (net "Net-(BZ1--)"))
 (segment (start 120.250 130.250) (end 120.750 129.750) (width 0.40) (layer "B.Cu") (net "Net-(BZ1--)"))
 (segment (start 120.750 129.750) (end 141.000 129.750) (width 0.40) (layer "B.Cu") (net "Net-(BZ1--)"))
 (segment (start 141.000 129.750) (end 141.500 129.250) (width 0.40) (layer "B.Cu") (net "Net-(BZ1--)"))
 (segment (start 141.500 129.250) (end 141.500 101.500) (width 0.40) (layer "B.Cu") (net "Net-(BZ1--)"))
 (segment (start 141.500 101.500) (end 141.000 101.000) (width 0.40) (layer "B.Cu") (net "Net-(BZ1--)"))
 (segment (start 141.000 101.000) (end 138.000 101.000) (width 0.40) (layer "B.Cu") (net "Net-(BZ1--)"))
 (segment (start 138.000 101.000) (end 137.500 101.500) (width 0.40) (layer "B.Cu") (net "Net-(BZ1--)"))
 (segment (start 137.500 101.500) (end 137.500 102.750) (width 0.40) (layer "B.Cu") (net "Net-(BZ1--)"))
 (segment (start 137.500 102.750) (end 136.040 102.750) (width 0.40) (layer "B.Cu") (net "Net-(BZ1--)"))
 (segment (start 136.040 102.750) (end 137.500 102.750) (width 0.40) (layer "B.Cu") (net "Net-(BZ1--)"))
 (segment (start 137.500 102.750) (end 137.500 101.500) (width 0.40) (layer "B.Cu") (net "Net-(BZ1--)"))
 (segment (start 137.500 101.500) (end 138.000 101.000) (width 0.40) (layer "B.Cu") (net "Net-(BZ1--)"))
 (segment (start 138.000 101.000) (end 141.000 101.000) (width 0.40) (layer "B.Cu") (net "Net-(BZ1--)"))
 (segment (start 141.000 101.000) (end 141.500 101.500) (width 0.40) (layer "B.Cu") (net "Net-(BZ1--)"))
 (segment (start 141.500 101.500) (end 141.500 111.200) (width 0.40) (layer "B.Cu") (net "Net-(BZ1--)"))
 (segment (start 141.500 111.200) (end 141.100 111.200) (width 0.40) (layer "B.Cu") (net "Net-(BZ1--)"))
 (segment (start 108.000 115.500) (end 106.000 115.500) (width 0.60) (layer "B.Cu") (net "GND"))
 (segment (start 106.000 115.500) (end 105.500 116.000) (width 0.60) (layer "B.Cu") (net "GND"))
 (segment (start 105.500 116.000) (end 105.500 120.750) (width 0.60) (layer "B.Cu") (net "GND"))
 (segment (start 105.500 120.750) (end 105.000 121.250) (width 0.60) (layer "B.Cu") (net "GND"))
 (segment (start 105.000 121.250) (end 104.000 121.250) (width 0.60) (layer "B.Cu") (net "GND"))
 (segment (start 104.000 121.250) (end 104.000 121.350) (width 0.60) (layer "B.Cu") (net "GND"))
 (segment (start 108.000 115.500) (end 111.500 115.500) (width 0.60) (layer "B.Cu") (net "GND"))
 (segment (start 111.500 115.500) (end 112.000 115.000) (width 0.60) (layer "B.Cu") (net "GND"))
 (segment (start 112.000 115.000) (end 112.000 110.750) (width 0.60) (layer "B.Cu") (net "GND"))
 (segment (start 112.000 110.750) (end 113.380 110.750) (width 0.60) (layer "B.Cu") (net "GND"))
 (segment (start 113.380 110.750) (end 113.380 110.650) (width 0.60) (layer "B.Cu") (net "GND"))
 (segment (start 129.890 103.000) (end 130.000 103.000) (width 0.60) (layer "B.Cu") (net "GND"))
 (segment (start 130.000 103.000) (end 130.000 102.250) (width 0.60) (layer "B.Cu") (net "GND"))
 (segment (start 130.000 102.250) (end 133.500 102.250) (width 0.60) (layer "B.Cu") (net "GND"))
 (segment (start 133.500 102.250) (end 133.500 102.800) (width 0.60) (layer "B.Cu") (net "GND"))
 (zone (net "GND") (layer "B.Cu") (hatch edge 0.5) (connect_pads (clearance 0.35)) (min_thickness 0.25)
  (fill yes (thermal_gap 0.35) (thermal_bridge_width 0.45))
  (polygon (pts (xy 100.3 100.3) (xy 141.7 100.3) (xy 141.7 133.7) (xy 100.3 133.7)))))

